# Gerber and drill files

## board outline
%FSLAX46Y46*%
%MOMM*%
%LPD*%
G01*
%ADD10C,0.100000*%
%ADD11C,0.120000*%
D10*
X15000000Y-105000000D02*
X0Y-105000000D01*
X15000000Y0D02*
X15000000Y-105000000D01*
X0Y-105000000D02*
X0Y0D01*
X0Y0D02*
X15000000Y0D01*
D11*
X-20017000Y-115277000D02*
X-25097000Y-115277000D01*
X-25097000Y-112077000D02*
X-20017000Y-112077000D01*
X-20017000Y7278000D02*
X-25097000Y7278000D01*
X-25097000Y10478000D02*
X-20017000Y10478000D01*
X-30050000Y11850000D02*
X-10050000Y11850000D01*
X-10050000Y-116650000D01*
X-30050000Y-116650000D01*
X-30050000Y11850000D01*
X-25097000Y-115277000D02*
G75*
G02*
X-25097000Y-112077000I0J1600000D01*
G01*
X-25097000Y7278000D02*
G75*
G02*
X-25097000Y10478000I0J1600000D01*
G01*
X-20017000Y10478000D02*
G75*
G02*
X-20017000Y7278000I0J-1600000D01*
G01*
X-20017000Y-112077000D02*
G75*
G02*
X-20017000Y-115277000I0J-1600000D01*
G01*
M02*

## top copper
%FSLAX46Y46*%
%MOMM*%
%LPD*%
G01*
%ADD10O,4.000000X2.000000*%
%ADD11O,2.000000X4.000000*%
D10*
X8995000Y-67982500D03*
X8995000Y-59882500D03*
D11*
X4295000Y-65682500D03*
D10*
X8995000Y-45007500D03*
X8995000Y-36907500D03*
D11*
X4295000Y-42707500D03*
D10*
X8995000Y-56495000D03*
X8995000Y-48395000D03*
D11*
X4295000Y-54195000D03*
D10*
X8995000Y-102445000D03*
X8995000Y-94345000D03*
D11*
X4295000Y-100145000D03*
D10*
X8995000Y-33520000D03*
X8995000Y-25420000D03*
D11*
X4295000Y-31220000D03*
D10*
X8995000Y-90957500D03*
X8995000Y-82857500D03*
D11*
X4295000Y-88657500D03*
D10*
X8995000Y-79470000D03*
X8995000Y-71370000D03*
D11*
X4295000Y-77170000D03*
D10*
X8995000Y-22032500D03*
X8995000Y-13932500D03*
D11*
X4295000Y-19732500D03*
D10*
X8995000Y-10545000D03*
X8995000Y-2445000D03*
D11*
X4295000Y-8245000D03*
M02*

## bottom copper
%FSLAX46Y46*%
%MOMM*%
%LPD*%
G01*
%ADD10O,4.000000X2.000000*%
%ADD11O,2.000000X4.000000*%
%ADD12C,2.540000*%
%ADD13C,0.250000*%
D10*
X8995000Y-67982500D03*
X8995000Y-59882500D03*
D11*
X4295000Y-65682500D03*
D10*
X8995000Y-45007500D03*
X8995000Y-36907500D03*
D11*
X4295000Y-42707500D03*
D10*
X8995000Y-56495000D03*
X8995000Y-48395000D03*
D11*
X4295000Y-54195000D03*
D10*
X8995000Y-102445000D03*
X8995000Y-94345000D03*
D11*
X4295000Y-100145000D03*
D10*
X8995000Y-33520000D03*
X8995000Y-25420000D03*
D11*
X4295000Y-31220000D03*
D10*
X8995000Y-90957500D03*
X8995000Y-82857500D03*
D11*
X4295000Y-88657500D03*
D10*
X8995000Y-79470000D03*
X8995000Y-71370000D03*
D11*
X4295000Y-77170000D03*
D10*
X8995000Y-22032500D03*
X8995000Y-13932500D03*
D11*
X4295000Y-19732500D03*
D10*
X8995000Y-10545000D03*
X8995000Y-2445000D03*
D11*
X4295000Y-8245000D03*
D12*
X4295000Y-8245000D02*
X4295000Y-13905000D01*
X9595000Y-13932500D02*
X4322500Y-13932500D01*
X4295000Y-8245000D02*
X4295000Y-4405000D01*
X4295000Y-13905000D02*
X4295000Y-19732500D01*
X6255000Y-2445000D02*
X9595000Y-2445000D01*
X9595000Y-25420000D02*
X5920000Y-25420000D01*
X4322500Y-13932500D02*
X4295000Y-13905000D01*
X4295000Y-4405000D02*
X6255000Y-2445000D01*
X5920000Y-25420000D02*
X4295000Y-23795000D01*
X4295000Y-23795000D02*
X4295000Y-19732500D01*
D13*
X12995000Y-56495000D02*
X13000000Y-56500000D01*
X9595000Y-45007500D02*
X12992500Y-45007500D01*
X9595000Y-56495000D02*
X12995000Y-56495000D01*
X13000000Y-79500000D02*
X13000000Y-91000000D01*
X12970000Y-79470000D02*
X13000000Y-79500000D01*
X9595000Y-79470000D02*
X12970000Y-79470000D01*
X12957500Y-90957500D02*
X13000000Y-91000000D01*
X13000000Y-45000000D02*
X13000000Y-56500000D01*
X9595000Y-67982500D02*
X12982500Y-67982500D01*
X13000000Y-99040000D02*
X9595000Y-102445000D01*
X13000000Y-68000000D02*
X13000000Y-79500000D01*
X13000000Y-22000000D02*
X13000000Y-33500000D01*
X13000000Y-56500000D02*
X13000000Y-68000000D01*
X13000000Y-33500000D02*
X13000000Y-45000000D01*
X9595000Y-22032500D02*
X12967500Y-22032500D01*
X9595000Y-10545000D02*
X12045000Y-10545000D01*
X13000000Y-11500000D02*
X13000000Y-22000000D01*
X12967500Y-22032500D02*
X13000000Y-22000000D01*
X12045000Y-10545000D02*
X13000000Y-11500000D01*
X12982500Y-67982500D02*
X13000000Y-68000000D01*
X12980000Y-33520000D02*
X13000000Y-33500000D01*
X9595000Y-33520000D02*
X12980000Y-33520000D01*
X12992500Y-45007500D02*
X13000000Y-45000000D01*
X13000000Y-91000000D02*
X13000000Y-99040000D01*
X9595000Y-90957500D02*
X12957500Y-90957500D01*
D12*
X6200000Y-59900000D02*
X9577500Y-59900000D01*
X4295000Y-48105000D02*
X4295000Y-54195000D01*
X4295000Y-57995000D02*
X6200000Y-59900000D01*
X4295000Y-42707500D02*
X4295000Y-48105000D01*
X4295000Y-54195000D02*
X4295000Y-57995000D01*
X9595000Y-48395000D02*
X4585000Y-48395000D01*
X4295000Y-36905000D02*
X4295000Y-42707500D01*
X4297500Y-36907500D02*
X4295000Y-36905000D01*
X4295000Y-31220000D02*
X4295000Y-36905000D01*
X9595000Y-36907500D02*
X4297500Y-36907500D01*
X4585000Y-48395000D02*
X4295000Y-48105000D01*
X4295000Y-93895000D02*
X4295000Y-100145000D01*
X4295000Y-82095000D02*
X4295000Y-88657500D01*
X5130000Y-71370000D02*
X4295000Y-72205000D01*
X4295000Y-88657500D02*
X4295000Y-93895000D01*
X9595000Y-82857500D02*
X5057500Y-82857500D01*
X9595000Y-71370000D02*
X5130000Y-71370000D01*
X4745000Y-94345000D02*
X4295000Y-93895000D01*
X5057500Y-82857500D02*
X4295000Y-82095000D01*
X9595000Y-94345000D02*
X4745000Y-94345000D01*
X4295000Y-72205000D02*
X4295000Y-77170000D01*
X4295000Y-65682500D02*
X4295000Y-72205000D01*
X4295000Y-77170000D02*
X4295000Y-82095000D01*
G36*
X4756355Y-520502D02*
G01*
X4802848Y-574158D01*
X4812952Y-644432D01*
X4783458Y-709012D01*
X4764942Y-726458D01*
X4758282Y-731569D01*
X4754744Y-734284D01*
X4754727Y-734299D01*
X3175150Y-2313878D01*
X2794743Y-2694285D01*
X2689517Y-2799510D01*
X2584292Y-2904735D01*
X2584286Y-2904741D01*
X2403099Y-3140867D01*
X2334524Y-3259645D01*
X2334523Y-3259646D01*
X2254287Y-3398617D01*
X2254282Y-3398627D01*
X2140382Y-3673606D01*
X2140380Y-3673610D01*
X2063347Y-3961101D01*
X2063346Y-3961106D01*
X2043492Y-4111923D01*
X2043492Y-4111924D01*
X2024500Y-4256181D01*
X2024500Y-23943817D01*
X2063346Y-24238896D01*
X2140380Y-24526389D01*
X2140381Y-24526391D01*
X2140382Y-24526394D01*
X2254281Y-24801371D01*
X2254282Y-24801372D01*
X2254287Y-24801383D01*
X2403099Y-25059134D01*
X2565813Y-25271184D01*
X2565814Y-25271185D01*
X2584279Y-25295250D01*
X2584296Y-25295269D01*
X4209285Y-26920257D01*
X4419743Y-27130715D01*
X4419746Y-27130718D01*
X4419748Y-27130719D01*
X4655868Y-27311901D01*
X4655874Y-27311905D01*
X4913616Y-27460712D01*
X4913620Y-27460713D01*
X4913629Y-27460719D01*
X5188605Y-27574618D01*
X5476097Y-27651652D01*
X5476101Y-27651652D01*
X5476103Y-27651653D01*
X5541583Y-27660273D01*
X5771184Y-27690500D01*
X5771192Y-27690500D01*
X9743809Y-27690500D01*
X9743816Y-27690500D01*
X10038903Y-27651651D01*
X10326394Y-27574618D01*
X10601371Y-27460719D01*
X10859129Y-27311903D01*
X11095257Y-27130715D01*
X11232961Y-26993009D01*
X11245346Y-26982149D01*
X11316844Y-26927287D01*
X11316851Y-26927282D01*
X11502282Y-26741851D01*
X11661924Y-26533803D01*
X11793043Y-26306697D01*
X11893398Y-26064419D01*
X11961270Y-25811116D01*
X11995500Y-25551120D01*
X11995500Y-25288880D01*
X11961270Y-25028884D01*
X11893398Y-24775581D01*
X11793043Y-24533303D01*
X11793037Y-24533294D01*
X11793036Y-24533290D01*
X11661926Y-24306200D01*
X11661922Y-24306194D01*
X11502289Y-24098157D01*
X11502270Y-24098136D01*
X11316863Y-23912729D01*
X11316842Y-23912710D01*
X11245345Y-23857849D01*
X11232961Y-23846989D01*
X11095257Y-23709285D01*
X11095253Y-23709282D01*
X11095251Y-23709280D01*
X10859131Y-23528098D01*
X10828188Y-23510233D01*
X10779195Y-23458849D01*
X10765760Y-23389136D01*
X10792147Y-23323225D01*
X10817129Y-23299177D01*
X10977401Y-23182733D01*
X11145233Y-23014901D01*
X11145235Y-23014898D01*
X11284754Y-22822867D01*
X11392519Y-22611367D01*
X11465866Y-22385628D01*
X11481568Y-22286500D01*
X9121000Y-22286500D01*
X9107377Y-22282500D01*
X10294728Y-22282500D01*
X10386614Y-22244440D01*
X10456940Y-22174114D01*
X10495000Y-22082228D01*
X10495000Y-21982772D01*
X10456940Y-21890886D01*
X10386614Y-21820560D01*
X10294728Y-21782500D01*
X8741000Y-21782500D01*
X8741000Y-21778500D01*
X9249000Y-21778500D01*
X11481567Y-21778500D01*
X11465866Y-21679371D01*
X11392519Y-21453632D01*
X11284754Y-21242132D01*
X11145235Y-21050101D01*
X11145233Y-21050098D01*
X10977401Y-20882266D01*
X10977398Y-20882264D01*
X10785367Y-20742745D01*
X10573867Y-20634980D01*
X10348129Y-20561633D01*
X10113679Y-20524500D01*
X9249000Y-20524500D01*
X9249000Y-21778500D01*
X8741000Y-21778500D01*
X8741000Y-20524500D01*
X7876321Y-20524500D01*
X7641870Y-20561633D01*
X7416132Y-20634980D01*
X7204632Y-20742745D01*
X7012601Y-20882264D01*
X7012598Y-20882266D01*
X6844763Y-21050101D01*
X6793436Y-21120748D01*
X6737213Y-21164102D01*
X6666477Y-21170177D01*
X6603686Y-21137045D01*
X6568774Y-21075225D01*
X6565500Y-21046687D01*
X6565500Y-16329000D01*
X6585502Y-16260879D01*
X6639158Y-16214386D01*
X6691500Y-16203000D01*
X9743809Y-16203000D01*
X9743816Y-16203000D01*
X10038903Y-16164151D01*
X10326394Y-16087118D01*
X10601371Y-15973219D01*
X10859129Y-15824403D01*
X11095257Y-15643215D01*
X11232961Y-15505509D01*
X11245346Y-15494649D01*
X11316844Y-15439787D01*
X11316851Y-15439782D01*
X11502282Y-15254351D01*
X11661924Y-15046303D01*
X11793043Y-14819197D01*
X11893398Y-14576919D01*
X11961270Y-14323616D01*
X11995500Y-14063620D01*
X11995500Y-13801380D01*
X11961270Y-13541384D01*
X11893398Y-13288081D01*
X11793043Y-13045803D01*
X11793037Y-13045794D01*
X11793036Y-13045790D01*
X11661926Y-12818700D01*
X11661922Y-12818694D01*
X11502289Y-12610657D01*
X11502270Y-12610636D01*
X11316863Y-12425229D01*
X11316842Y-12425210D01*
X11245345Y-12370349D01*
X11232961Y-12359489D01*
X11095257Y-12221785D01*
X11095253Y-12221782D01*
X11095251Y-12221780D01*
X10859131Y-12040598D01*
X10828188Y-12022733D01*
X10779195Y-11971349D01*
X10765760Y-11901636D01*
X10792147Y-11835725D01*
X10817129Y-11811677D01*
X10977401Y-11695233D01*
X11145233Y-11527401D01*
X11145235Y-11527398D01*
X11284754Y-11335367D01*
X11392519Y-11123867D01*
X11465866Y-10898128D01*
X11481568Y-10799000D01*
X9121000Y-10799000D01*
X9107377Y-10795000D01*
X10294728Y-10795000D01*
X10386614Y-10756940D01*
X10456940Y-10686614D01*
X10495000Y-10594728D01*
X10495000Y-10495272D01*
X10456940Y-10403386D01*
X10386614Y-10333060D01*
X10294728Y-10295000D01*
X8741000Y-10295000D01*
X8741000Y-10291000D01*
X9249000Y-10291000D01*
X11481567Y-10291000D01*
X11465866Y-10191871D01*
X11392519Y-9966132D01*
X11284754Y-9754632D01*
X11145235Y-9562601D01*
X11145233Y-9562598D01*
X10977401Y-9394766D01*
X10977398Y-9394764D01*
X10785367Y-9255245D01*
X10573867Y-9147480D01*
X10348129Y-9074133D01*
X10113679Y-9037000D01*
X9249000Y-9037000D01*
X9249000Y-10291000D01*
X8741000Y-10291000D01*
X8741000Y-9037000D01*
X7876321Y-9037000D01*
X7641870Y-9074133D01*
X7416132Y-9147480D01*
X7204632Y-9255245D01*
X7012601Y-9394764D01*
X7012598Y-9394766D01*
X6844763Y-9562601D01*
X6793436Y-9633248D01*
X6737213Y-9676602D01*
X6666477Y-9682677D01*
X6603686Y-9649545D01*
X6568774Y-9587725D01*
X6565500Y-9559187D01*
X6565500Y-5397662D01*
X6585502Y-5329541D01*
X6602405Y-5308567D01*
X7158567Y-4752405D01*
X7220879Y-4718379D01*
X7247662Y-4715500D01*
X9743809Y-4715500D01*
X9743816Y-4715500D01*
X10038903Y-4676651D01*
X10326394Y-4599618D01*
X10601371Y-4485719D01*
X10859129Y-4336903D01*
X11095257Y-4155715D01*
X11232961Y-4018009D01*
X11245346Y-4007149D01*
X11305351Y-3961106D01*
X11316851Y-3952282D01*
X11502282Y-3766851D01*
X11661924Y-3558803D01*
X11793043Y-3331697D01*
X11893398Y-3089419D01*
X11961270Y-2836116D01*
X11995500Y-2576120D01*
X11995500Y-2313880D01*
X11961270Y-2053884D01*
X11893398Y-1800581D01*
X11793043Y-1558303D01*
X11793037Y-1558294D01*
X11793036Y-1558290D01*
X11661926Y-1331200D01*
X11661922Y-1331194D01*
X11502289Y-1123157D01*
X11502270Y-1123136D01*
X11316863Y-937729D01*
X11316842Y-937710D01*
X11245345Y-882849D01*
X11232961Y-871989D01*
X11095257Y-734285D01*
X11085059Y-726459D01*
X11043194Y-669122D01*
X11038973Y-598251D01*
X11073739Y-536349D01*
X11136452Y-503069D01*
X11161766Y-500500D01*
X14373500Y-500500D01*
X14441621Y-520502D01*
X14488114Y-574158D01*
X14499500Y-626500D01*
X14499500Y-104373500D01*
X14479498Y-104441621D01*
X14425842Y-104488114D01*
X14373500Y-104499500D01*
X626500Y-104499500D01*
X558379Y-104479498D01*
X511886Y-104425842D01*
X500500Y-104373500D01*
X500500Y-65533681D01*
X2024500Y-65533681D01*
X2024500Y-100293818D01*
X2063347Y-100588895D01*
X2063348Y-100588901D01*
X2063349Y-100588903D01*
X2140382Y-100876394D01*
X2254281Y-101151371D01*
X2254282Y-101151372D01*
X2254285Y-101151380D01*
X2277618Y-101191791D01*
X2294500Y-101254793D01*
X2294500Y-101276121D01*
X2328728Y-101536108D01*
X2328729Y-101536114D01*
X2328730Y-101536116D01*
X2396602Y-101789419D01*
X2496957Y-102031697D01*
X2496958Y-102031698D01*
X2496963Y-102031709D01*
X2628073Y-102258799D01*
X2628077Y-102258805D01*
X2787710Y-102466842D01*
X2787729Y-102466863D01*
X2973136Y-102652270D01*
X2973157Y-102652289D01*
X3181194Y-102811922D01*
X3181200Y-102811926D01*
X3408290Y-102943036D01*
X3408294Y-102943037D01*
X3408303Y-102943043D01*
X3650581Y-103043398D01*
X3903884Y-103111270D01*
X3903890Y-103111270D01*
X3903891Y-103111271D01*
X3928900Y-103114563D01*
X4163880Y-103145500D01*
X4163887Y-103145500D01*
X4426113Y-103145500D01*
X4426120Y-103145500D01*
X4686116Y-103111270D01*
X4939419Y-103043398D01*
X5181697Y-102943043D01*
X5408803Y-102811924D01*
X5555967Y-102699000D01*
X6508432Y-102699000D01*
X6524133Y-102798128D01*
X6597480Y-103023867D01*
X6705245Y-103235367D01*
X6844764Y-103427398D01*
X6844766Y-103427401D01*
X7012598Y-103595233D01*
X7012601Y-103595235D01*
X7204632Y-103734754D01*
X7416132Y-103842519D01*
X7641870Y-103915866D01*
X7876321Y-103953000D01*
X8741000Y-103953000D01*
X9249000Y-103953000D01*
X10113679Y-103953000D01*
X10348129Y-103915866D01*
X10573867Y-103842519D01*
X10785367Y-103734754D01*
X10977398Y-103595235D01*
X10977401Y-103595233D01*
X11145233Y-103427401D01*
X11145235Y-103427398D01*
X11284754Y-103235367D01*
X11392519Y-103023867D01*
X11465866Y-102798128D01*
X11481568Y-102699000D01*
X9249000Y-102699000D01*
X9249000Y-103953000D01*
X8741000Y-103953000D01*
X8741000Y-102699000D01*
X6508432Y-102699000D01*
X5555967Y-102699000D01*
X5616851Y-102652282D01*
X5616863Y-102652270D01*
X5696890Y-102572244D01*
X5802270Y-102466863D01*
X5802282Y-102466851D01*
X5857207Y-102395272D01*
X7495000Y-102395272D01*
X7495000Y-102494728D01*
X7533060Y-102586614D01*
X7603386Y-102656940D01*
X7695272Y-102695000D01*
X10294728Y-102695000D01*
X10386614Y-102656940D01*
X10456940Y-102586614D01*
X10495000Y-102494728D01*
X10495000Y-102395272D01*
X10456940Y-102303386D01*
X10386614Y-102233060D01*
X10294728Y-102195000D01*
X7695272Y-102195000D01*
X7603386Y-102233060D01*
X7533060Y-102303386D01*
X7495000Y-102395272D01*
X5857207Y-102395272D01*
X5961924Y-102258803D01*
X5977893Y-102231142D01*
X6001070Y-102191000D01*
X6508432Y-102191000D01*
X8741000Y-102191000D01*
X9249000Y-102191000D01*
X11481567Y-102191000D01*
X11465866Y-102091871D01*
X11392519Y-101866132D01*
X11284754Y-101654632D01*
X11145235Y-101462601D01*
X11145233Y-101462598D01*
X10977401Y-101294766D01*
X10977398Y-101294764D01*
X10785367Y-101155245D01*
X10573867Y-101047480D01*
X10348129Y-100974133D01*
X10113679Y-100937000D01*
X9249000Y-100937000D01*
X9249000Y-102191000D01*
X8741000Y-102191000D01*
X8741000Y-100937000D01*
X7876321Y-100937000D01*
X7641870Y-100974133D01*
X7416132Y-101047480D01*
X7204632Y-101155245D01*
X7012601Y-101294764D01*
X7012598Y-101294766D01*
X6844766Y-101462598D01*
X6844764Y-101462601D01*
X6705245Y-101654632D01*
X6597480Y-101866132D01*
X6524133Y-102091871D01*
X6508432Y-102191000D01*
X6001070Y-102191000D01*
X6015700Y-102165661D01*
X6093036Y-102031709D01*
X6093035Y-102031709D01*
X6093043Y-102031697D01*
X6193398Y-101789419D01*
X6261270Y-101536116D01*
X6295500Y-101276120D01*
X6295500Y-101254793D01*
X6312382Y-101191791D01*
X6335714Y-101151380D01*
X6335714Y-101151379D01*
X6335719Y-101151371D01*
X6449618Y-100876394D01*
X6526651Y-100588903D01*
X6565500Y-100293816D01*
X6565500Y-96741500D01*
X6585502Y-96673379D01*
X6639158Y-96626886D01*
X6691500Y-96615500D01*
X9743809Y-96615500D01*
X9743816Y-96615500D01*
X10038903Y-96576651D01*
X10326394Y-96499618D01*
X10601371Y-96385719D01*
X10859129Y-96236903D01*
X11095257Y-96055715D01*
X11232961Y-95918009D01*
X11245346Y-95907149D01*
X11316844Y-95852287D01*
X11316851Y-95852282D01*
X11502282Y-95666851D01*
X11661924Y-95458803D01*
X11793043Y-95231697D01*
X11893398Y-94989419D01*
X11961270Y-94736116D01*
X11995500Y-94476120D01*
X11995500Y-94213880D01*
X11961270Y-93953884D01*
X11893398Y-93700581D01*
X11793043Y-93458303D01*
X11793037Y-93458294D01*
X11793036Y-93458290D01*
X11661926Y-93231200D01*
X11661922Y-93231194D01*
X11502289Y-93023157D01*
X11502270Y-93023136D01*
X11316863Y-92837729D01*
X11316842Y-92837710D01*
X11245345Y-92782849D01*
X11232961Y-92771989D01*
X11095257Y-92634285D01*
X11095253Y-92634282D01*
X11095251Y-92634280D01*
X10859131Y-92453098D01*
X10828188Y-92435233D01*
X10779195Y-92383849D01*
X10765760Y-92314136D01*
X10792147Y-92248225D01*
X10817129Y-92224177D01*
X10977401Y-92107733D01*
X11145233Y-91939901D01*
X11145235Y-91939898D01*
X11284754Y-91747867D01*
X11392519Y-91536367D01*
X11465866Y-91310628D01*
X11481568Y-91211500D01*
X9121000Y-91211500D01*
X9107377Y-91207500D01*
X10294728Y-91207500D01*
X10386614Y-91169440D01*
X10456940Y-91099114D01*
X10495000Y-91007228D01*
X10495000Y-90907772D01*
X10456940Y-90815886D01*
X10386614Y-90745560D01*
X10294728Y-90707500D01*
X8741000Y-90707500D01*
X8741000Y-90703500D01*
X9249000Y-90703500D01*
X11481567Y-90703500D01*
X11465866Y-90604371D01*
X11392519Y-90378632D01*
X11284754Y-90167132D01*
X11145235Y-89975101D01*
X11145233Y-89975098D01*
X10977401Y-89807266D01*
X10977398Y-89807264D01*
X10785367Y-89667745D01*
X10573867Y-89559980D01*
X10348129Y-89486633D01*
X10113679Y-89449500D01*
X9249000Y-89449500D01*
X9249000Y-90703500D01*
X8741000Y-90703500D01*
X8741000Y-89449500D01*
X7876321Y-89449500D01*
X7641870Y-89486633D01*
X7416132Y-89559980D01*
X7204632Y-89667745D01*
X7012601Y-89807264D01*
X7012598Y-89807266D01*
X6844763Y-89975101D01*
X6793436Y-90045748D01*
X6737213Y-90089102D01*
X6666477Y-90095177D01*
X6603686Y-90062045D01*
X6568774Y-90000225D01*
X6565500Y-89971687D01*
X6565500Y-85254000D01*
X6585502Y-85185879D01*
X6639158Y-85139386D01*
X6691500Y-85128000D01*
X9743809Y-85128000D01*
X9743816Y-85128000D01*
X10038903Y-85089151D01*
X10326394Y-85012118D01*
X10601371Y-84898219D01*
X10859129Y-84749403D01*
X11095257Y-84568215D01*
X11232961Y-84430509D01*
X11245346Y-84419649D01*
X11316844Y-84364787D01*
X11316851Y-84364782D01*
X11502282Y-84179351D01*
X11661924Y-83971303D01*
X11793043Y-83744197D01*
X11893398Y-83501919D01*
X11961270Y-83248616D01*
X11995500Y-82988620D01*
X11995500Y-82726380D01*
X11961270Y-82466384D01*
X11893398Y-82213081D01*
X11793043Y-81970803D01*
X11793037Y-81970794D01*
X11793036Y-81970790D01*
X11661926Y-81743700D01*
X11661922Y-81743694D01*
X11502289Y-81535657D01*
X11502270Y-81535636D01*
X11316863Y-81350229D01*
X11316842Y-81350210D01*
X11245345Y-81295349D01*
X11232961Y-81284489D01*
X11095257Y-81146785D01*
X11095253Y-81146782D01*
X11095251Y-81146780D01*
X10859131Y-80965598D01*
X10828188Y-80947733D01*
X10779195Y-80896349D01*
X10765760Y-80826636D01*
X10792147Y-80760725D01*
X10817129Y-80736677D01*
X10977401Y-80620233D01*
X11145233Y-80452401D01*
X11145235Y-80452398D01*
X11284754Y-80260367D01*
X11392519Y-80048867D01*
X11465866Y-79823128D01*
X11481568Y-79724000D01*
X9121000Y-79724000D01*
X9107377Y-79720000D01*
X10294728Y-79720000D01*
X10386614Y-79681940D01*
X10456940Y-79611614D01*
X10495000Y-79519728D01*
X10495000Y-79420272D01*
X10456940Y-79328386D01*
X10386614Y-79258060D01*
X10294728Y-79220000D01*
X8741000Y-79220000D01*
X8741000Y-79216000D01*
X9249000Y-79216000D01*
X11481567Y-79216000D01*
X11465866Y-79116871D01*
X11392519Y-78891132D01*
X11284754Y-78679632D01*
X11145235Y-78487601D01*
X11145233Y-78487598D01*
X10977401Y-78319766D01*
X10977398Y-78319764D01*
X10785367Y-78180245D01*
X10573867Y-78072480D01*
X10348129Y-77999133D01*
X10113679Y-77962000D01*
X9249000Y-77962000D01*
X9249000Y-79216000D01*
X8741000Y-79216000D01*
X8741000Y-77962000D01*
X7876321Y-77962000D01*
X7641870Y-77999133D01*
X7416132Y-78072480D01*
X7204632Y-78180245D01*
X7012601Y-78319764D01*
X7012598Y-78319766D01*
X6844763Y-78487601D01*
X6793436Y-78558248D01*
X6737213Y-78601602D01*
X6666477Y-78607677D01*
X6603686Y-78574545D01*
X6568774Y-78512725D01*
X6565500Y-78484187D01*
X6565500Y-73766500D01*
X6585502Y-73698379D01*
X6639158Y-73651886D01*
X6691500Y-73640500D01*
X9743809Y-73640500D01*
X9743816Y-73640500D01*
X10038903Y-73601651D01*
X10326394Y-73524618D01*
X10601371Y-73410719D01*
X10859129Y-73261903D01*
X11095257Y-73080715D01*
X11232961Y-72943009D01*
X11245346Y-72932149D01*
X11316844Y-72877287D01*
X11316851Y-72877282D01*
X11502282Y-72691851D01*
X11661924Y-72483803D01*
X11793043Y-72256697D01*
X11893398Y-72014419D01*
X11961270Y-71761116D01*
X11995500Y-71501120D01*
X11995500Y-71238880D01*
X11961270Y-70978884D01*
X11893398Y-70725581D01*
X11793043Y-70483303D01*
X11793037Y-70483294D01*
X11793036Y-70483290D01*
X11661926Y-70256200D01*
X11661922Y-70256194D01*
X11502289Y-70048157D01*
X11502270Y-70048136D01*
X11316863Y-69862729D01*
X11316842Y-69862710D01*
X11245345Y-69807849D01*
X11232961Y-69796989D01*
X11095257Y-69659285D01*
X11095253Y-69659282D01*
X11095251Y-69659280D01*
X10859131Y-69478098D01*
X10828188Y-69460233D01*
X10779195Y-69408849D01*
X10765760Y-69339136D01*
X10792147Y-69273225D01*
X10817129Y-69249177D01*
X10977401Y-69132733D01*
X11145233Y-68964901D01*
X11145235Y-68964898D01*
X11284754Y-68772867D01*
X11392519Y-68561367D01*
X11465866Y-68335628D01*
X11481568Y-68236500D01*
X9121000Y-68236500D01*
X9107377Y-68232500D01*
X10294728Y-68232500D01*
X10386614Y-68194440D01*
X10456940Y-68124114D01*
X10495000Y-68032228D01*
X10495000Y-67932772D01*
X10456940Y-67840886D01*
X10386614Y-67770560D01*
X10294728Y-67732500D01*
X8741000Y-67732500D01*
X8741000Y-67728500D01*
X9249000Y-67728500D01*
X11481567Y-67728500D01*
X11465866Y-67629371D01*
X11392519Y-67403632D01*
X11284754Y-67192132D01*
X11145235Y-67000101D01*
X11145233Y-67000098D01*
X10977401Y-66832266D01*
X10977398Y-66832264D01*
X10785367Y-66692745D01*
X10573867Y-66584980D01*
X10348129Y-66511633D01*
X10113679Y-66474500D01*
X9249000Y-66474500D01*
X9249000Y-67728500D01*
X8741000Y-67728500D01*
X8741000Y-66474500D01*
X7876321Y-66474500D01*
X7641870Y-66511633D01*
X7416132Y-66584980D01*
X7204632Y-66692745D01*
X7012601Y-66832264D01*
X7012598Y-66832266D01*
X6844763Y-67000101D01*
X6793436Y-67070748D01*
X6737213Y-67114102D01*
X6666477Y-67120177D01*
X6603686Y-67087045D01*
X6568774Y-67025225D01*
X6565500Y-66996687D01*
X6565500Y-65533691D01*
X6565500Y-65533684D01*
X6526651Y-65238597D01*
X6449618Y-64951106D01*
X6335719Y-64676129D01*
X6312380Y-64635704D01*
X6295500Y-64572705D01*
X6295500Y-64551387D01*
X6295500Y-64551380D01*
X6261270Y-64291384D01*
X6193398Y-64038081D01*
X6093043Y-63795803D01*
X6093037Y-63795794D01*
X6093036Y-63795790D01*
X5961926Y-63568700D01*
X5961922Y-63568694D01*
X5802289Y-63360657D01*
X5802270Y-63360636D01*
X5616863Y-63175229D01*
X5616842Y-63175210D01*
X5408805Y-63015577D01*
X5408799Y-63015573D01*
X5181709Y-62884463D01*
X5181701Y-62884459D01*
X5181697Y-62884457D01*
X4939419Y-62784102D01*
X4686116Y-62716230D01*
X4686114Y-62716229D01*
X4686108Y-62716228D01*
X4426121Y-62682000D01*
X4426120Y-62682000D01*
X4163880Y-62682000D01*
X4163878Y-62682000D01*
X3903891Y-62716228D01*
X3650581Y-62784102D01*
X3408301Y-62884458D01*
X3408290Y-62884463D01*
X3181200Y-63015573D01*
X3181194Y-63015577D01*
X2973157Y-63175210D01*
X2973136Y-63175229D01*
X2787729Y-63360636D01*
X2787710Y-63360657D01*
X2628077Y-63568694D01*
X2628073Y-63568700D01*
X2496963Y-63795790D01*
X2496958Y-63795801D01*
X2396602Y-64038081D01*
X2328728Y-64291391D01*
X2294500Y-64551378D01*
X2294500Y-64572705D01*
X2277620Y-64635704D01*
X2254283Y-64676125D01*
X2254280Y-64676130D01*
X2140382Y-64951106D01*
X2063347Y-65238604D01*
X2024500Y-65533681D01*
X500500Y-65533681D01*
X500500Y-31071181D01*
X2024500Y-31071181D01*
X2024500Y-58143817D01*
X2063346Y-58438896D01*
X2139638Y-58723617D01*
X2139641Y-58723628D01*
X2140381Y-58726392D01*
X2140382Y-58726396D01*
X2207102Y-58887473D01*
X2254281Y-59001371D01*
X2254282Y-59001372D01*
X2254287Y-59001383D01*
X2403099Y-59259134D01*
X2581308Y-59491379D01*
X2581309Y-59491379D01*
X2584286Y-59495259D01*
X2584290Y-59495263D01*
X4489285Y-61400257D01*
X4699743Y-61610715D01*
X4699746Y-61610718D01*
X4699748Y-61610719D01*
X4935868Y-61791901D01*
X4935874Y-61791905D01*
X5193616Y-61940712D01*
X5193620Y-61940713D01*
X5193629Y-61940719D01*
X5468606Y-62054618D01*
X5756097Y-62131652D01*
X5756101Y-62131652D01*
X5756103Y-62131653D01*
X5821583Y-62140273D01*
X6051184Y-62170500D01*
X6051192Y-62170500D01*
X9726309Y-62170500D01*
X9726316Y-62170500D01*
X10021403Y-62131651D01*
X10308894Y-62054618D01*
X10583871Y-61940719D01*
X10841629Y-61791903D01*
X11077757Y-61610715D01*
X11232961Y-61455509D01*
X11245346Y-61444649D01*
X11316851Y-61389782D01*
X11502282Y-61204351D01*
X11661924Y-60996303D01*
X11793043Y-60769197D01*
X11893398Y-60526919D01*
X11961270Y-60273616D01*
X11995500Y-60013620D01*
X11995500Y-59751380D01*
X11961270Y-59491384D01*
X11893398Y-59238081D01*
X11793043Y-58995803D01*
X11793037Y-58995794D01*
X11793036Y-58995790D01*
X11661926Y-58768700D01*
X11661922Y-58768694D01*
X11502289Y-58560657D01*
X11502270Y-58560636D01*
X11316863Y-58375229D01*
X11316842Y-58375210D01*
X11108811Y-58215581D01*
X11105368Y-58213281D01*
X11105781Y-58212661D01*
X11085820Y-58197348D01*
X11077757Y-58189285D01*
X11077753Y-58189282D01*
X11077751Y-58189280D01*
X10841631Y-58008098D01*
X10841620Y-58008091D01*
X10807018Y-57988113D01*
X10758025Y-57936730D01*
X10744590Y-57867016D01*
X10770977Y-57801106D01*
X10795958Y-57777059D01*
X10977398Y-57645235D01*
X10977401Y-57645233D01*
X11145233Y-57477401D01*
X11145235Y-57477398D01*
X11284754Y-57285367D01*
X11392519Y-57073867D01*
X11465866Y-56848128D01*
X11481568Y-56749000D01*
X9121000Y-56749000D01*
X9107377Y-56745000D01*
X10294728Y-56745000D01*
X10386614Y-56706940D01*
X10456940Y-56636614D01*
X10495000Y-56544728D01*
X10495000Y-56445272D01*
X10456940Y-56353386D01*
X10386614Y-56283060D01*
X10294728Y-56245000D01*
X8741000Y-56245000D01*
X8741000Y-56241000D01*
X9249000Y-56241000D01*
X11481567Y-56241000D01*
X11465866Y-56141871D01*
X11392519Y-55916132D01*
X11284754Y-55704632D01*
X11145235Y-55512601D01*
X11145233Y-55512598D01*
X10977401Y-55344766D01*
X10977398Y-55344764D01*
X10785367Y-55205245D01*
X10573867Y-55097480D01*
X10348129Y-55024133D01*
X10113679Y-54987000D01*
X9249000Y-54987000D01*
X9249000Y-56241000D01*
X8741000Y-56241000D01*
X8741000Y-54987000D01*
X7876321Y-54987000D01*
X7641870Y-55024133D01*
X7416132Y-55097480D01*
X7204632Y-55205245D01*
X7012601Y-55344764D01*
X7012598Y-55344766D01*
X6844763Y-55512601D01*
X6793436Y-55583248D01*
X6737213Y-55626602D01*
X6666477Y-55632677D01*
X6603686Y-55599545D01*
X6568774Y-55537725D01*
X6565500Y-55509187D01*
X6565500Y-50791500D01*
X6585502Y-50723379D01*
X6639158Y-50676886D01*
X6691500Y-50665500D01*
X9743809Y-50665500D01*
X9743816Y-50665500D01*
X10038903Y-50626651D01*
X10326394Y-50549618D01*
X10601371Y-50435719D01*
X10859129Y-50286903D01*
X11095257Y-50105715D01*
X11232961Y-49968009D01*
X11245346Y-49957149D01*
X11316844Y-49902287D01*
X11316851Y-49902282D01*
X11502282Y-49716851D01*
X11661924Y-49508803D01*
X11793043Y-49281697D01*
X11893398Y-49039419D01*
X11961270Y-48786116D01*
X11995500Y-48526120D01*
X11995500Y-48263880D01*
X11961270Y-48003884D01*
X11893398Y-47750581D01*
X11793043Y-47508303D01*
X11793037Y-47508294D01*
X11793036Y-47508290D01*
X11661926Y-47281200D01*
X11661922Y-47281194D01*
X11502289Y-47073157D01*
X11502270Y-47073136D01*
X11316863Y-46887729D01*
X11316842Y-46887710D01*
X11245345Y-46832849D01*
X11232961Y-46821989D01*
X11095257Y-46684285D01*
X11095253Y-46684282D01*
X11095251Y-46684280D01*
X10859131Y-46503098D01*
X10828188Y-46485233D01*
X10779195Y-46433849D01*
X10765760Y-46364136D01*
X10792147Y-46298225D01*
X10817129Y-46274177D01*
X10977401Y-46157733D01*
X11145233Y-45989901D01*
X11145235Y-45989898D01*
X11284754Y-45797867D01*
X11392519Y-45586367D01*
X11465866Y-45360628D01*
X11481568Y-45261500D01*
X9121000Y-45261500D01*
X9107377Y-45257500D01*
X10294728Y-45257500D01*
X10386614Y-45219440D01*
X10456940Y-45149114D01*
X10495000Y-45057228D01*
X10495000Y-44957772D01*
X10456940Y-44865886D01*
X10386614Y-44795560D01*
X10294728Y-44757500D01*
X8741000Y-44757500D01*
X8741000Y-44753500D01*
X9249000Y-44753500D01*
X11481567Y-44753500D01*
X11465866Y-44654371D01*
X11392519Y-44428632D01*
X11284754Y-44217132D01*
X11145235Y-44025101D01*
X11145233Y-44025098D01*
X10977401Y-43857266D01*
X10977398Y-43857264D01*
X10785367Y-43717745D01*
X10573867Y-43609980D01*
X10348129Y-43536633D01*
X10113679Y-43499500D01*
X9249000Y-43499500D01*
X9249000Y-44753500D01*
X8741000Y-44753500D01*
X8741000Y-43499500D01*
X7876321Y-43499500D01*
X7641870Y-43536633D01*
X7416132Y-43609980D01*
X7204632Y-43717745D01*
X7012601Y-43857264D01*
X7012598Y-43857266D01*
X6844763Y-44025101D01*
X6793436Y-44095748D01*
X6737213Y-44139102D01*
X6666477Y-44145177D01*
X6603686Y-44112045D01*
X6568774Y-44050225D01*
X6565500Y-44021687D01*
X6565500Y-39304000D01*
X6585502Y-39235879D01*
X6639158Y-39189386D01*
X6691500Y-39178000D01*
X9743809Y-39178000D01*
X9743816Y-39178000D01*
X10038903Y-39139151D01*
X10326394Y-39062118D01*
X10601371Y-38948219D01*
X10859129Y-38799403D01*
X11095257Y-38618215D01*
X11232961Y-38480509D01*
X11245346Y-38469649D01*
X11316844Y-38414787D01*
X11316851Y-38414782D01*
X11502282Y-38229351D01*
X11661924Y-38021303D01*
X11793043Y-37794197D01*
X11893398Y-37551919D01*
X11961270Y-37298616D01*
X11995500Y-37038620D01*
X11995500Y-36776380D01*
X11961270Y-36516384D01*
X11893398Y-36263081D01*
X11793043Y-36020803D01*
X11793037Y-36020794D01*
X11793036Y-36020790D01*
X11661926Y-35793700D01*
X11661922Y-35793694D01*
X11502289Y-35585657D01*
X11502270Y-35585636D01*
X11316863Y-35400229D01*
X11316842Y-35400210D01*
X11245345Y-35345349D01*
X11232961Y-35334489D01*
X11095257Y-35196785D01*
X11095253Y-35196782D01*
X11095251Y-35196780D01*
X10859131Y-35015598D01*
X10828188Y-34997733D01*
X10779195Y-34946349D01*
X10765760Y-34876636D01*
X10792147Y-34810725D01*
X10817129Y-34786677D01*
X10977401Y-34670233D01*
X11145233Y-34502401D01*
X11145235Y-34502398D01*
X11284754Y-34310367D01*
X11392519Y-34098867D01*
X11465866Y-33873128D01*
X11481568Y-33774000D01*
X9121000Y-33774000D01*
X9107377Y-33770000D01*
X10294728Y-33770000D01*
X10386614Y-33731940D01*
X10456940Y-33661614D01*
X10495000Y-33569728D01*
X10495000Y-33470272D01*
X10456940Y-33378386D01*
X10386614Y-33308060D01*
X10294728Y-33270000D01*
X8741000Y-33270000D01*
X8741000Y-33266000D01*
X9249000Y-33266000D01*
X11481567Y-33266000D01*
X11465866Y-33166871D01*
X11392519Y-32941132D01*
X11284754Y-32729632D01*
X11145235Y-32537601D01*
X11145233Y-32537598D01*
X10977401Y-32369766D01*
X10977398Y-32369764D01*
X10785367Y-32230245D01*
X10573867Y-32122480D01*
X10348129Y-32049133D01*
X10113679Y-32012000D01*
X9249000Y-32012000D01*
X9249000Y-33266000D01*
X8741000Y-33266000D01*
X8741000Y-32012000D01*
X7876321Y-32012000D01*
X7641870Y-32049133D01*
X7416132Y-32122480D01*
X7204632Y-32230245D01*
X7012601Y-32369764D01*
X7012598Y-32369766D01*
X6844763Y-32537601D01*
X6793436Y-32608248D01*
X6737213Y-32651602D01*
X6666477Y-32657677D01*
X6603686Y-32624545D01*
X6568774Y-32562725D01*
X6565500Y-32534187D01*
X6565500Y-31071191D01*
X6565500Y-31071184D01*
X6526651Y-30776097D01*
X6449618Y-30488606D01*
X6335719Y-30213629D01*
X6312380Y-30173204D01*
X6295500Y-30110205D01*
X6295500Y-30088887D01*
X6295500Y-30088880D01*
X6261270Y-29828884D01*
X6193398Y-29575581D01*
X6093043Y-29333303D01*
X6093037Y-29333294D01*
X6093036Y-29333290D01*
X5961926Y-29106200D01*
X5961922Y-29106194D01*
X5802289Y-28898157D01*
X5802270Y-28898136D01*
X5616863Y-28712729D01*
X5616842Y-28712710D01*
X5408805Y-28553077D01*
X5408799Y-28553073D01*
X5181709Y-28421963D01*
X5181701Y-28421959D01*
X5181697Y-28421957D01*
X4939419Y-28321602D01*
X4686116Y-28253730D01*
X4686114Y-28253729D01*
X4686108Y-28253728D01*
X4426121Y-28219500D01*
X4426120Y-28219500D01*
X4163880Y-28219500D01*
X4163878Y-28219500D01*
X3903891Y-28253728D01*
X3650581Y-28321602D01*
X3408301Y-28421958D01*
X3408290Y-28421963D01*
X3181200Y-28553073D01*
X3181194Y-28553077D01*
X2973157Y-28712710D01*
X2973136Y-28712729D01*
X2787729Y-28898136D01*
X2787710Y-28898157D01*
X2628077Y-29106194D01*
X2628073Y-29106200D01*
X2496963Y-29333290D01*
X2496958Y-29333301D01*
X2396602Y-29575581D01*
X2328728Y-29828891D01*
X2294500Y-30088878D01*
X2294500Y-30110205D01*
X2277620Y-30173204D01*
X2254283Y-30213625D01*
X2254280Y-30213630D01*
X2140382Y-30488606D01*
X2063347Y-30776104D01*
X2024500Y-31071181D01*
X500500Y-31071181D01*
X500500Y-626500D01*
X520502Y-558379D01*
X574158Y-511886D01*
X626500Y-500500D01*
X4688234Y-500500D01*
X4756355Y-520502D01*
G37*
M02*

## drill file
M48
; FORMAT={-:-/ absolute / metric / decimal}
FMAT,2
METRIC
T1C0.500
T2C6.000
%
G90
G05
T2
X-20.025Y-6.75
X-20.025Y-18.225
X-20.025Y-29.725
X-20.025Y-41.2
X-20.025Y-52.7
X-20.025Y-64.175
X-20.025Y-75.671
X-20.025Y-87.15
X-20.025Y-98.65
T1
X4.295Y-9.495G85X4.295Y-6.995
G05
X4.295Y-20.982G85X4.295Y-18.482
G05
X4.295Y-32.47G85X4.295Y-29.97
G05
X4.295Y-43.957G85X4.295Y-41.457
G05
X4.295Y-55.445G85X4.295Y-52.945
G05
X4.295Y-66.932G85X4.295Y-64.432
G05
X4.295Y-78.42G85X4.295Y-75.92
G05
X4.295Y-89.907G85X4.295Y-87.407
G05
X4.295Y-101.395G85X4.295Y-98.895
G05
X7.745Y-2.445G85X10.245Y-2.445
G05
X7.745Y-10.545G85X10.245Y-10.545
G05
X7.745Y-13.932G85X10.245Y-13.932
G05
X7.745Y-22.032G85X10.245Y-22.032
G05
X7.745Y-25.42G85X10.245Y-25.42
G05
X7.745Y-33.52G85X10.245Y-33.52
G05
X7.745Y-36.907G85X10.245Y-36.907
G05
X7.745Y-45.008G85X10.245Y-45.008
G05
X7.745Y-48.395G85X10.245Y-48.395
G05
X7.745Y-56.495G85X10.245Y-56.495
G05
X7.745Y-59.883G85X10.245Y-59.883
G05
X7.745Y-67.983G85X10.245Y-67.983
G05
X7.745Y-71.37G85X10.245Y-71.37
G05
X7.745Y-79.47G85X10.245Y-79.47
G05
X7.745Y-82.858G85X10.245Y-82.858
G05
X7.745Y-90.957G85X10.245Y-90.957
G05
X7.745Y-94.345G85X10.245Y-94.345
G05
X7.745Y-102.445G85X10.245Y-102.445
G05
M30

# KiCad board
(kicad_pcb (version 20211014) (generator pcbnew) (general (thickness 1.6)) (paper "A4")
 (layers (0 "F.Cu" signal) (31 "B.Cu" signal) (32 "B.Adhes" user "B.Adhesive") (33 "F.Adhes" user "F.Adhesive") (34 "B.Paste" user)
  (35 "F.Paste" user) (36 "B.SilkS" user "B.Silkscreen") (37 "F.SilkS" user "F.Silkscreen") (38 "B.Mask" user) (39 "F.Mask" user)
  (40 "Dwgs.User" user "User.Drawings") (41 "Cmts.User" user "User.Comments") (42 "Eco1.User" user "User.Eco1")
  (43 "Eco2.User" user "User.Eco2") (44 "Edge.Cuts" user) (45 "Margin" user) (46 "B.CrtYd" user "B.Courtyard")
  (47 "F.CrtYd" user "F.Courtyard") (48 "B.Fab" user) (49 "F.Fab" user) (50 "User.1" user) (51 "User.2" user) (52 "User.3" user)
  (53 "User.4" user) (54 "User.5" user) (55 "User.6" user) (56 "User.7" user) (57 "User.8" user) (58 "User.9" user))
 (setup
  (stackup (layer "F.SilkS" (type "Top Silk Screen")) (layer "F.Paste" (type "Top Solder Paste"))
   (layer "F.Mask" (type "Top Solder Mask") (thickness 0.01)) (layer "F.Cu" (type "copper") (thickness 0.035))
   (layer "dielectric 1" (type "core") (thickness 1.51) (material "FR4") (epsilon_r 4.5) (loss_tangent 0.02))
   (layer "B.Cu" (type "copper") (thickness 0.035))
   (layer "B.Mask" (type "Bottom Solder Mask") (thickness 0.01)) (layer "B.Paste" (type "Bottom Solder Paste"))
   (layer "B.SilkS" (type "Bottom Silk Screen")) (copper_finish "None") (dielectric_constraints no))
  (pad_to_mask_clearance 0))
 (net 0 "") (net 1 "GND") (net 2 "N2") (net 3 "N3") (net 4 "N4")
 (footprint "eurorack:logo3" (layer "F.Cu") (at -25.575 54.775 90)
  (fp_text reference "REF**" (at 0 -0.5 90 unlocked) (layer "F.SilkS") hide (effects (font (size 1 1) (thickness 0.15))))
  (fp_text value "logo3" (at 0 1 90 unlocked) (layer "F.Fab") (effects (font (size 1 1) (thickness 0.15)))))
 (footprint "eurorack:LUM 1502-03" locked (layer "F.Cu") (at 2.895 58.4825)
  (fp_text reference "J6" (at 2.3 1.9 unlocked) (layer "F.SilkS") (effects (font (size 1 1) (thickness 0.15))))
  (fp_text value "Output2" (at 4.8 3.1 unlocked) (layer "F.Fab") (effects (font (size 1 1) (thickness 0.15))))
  (pad "S" thru_hole oval locked (at 6.1 9.5) (size 4 2) (drill oval 3 0.5) (layers *.Cu *.Mask) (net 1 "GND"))
  (pad "T" thru_hole oval locked (at 6.1 1.4) (size 4 2) (drill oval 3 0.5) (layers *.Cu *.Mask) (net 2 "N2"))
  (pad "TN" thru_hole oval locked (at 1.4 7.2 90) (size 4 2) (drill oval 3 0.5) (layers *.Cu *.Mask) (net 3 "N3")))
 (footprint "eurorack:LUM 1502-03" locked (layer "F.Cu") (at 2.895 35.5075)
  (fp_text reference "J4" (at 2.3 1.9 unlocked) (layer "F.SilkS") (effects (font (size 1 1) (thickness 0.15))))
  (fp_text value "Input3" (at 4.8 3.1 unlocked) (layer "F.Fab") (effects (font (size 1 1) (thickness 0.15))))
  (pad "S" thru_hole oval locked (at 6.1 9.5) (size 4 2) (drill oval 3 0.5) (layers *.Cu *.Mask) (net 1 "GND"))
  (pad "T" thru_hole oval locked (at 6.1 1.4) (size 4 2) (drill oval 3 0.5) (layers *.Cu *.Mask) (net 2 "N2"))
  (pad "TN" thru_hole oval locked (at 1.4 7.2 90) (size 4 2) (drill oval 3 0.5) (layers *.Cu *.Mask) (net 2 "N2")))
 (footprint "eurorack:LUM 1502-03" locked (layer "F.Cu") (at 2.895 46.995)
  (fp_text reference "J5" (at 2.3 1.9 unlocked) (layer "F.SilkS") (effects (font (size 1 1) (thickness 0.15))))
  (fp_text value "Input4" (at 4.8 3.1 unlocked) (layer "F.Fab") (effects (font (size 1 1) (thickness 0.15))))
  (pad "S" thru_hole oval locked (at 6.1 9.5) (size 4 2) (drill oval 3 0.5) (layers *.Cu *.Mask) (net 1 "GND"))
  (pad "T" thru_hole oval locked (at 6.1 1.4) (size 4 2) (drill oval 3 0.5) (layers *.Cu *.Mask) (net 2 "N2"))
  (pad "TN" thru_hole oval locked (at 1.4 7.2 90) (size 4 2) (drill oval 3 0.5) (layers *.Cu *.Mask) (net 2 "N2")))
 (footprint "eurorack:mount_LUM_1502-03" (layer "F.Cu") (at -20.025 41.2)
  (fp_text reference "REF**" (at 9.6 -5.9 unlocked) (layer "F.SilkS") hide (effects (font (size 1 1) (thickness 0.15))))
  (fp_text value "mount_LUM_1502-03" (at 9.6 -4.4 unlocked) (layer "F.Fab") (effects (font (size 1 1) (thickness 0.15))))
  (pad "" np_thru_hole circle (at 0 0) (size 6 6) (drill 6) (layers F&B.Cu *.Mask)))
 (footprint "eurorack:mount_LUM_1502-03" (layer "F.Cu") (at -20.025 52.7)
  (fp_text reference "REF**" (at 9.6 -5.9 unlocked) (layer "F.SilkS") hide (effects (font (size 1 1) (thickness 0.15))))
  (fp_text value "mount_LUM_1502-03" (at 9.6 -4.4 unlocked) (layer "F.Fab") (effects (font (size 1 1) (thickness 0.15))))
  (pad "" np_thru_hole circle (at 0 0) (size 6 6) (drill 6) (layers F&B.Cu *.Mask)))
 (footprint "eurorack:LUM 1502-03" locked (layer "F.Cu") (at 2.895 92.945)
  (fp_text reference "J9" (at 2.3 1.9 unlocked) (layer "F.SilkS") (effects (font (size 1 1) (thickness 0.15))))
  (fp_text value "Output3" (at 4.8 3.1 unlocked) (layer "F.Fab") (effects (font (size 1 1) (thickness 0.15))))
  (pad "S" thru_hole oval locked (at 6.1 9.5) (size 4 2) (drill oval 3 0.5) (layers *.Cu *.Mask) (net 1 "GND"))
  (pad "T" thru_hole oval locked (at 6.1 1.4) (size 4 2) (drill oval 3 0.5) (layers *.Cu *.Mask) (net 3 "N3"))
  (pad "TN" thru_hole oval locked (at 1.4 7.2 90) (size 4 2) (drill oval 3 0.5) (layers *.Cu *.Mask) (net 3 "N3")))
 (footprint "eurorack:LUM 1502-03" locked (layer "F.Cu") (at 2.895 24.02)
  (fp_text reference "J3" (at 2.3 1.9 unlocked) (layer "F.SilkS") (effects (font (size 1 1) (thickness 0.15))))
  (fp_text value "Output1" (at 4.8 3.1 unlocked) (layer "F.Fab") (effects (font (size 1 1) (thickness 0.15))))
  (pad "S" thru_hole oval locked (at 6.1 9.5) (size 4 2) (drill oval 3 0.5) (layers *.Cu *.Mask) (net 1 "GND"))
  (pad "T" thru_hole oval locked (at 6.1 1.4) (size 4 2) (drill oval 3 0.5) (layers *.Cu *.Mask) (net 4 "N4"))
  (pad "TN" thru_hole oval locked (at 1.4 7.2 90) (size 4 2) (drill oval 3 0.5) (layers *.Cu *.Mask) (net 2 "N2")))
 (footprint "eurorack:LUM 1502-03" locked (layer "F.Cu") (at 2.895 81.4575)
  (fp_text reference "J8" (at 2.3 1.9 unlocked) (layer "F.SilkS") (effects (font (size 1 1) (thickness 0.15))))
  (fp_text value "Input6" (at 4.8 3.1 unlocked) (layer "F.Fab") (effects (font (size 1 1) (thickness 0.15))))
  (pad "S" thru_hole oval locked (at 6.1 9.5) (size 4 2) (drill oval 3 0.5) (layers *.Cu *.Mask) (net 1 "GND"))
  (pad "T" thru_hole oval locked (at 6.1 1.4) (size 4 2) (drill oval 3 0.5) (layers *.Cu *.Mask) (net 3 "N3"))
  (pad "TN" thru_hole oval locked (at 1.4 7.2 90) (size 4 2) (drill oval 3 0.5) (layers *.Cu *.Mask) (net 3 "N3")))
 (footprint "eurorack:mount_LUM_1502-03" (layer "F.Cu") (at -20.025 64.175)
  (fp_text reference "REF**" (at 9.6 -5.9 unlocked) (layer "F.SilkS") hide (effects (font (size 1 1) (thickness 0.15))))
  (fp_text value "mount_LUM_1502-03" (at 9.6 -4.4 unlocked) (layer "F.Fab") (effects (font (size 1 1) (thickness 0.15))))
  (pad "" np_thru_hole circle (at 0 0) (size 6 6) (drill 6) (layers F&B.Cu *.Mask)))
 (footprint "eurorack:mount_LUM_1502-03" (layer "F.Cu") (at -20.025 6.75)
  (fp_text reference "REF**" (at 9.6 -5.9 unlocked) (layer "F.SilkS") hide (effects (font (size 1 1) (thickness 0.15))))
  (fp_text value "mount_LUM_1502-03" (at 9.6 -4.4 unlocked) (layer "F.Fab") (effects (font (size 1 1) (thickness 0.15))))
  (pad "" np_thru_hole circle (at 0 0) (size 6 6) (drill 6) (layers F&B.Cu *.Mask)))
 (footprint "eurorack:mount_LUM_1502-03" (layer "F.Cu") (at -20.025 75.671059)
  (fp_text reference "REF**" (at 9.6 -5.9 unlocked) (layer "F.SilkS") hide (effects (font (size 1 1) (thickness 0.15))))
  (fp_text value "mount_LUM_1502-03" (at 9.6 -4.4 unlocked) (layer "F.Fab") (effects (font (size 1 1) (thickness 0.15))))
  (pad "" np_thru_hole circle (at 0 0) (size 6 6) (drill 6) (layers F&B.Cu *.Mask)))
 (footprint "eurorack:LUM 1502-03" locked (layer "F.Cu") (at 2.895 69.97)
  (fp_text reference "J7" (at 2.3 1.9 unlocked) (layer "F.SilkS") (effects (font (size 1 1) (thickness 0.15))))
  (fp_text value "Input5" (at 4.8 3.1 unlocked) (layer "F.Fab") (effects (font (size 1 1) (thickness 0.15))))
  (pad "S" thru_hole oval locked (at 6.1 9.5) (size 4 2) (drill oval 3 0.5) (layers *.Cu *.Mask) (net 1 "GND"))
  (pad "T" thru_hole oval locked (at 6.1 1.4) (size 4 2) (drill oval 3 0.5) (layers *.Cu *.Mask) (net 3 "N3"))
  (pad "TN" thru_hole oval locked (at 1.4 7.2 90) (size 4 2) (drill oval 3 0.5) (layers *.Cu *.Mask) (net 3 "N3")))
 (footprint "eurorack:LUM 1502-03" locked (layer "F.Cu") (at 2.895 12.5325)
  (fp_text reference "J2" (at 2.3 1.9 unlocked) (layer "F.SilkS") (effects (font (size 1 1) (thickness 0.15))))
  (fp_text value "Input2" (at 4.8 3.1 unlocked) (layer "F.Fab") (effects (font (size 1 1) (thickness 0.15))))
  (pad "S" thru_hole oval locked (at 6.1 9.5) (size 4 2) (drill oval 3 0.5) (layers *.Cu *.Mask) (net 1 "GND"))
  (pad "T" thru_hole oval locked (at 6.1 1.4) (size 4 2) (drill oval 3 0.5) (layers *.Cu *.Mask) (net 4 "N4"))
  (pad "TN" thru_hole oval locked (at 1.4 7.2 90) (size 4 2) (drill oval 3 0.5) (layers *.Cu *.Mask) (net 4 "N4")))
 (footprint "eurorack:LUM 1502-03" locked (layer "F.Cu") (at 2.895 1.045)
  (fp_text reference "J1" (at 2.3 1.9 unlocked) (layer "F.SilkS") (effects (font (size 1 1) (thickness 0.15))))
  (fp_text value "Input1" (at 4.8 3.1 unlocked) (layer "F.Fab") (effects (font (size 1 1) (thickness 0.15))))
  (pad "S" thru_hole oval locked (at 6.1 9.5) (size 4 2) (drill oval 3 0.5) (layers *.Cu *.Mask) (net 1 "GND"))
  (pad "T" thru_hole oval locked (at 6.1 1.4) (size 4 2) (drill oval 3 0.5) (layers *.Cu *.Mask) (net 4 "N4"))
  (pad "TN" thru_hole oval locked (at 1.4 7.2 90) (size 4 2) (drill oval 3 0.5) (layers *.Cu *.Mask) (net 4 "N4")))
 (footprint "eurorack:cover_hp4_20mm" (layer "F.Cu") (at -30.05 -11.85)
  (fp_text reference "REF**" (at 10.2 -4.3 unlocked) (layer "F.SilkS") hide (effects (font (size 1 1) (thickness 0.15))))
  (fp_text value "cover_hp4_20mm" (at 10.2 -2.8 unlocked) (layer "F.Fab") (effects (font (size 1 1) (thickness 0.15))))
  (fp_line (start 10.033 127.127) (end 4.953 127.127) (layer "Edge.Cuts") (width 0.12))
  (fp_line (start 4.953 123.927) (end 10.033 123.927) (layer "Edge.Cuts") (width 0.12))
  (fp_line (start 10.033 4.572) (end 4.953 4.572) (layer "Edge.Cuts") (width 0.12))
  (fp_line (start 4.953 1.372) (end 10.033 1.372) (layer "Edge.Cuts") (width 0.12))
  (fp_rect (start 0 0) (end 20 128.5) (layer "Edge.Cuts") (width 0.12) (fill none))
  (fp_arc (start 4.953 127.127) (mid 3.353 125.527) (end 4.953 123.927) (layer "Edge.Cuts") (width 0.12))
  (fp_arc (start 4.953 4.572) (mid 3.353 2.972) (end 4.953 1.372) (layer "Edge.Cuts") (width 0.12))
  (fp_arc (start 10.033 1.372) (mid 11.633 2.972) (end 10.033 4.572) (layer "Edge.Cuts") (width 0.12))
  (fp_arc (start 10.033 123.927) (mid 11.633 125.527) (end 10.033 127.127) (layer "Edge.Cuts") (width 0.12)))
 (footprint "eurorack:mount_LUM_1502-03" (layer "F.Cu") (at -20.025 98.65)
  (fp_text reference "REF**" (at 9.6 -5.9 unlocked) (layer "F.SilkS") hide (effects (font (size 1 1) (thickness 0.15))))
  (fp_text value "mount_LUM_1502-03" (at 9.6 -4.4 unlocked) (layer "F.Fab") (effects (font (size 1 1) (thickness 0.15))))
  (pad "" np_thru_hole circle (at 0 0) (size 6 6) (drill 6) (layers F&B.Cu *.Mask)))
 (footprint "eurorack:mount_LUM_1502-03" (layer "F.Cu") (at -20.025 18.225)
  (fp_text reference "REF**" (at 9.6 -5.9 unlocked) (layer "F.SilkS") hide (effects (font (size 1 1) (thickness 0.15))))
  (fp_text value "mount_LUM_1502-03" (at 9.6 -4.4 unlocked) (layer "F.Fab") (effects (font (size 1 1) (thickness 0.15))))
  (pad "" np_thru_hole circle (at 0 0) (size 6 6) (drill 6) (layers F&B.Cu *.Mask)))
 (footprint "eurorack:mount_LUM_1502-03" (layer "F.Cu") (at -20.025 87.15)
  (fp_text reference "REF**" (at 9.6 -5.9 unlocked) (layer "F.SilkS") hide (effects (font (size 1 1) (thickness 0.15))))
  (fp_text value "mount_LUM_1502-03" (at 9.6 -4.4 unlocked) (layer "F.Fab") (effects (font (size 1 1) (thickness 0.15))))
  (pad "" np_thru_hole circle (at 0 0) (size 6 6) (drill 6) (layers F&B.Cu *.Mask)))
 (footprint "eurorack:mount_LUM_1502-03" (layer "F.Cu") (at -20.025 29.725)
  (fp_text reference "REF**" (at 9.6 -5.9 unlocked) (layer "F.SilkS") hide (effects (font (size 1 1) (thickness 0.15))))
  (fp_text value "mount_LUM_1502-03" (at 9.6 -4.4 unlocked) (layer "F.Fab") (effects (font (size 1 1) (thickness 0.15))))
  (pad "" np_thru_hole circle (at 0 0) (size 6 6) (drill 6) (layers F&B.Cu *.Mask)))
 (gr_line locked (start 15 105) (end 0 105) (layer "Edge.Cuts") (width 0.1))
 (gr_line locked (start 15 0) (end 15 105) (layer "Edge.Cuts") (width 0.1))
 (gr_line locked (start 0 105) (end 0 0) (layer "Edge.Cuts") (width 0.1))
 (gr_line locked (start 0 0) (end 15 0) (layer "Edge.Cuts") (width 0.1))
 (segment locked (start 4.295 8.245) (end 4.295 13.905) (width 2.54) (layer "B.Cu") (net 4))
 (segment locked (start 9.595 13.9325) (end 4.3225 13.9325) (width 2.54) (layer "B.Cu") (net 4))
 (segment locked (start 4.295 8.245) (end 4.295 4.405) (width 2.54) (layer "B.Cu") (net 4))
 (segment locked (start 4.295 13.905) (end 4.295 19.7325) (width 2.54) (layer "B.Cu") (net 4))
 (segment locked (start 6.255 2.445) (end 9.595 2.445) (width 2.54) (layer "B.Cu") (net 4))
 (segment locked (start 9.595 25.42) (end 5.92 25.42) (width 2.54) (layer "B.Cu") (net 4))
 (segment locked (start 4.3225 13.9325) (end 4.295 13.905) (width 2.54) (layer "B.Cu") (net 4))
 (segment locked (start 4.295 4.405) (end 6.255 2.445) (width 2.54) (layer "B.Cu") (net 4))
 (segment locked (start 5.92 25.42) (end 4.295 23.795) (width 2.54) (layer "B.Cu") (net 4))
 (segment locked (start 4.295 23.795) (end 4.295 19.7325) (width 2.54) (layer "B.Cu") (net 4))
 (segment locked (start 12.995 56.495) (end 13 56.5) (width 0.25) (layer "B.Cu") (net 1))
 (segment locked (start 9.595 45.0075) (end 12.9925 45.0075) (width 0.25) (layer "B.Cu") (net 1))
 (segment locked (start 9.595 56.495) (end 12.995 56.495) (width 0.25) (layer "B.Cu") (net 1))
 (segment locked (start 13 79.5) (end 13 91) (width 0.25) (layer "B.Cu") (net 1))
 (segment locked (start 12.97 79.47) (end 13 79.5) (width 0.25) (layer "B.Cu") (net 1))
 (segment locked (start 9.595 79.47) (end 12.97 79.47) (width 0.25) (layer "B.Cu") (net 1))
 (segment locked (start 12.9575 90.9575) (end 13 91) (width 0.25) (layer "B.Cu") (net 1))
 (segment locked (start 13 45) (end 13 56.5) (width 0.25) (layer "B.Cu") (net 1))
 (segment locked (start 9.595 67.9825) (end 12.9825 67.9825) (width 0.25) (layer "B.Cu") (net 1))
 (segment locked (start 13 99.04) (end 9.595 102.445) (width 0.25) (layer "B.Cu") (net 1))
 (segment locked (start 13 68) (end 13 79.5) (width 0.25) (layer "B.Cu") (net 1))
 (segment locked (start 13 22) (end 13 33.5) (width 0.25) (layer "B.Cu") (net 1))
 (segment locked (start 13 56.5) (end 13 68) (width 0.25) (layer "B.Cu") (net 1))
 (segment locked (start 13 33.5) (end 13 45) (width 0.25) (layer "B.Cu") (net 1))
 (segment locked (start 9.595 22.0325) (end 12.9675 22.0325) (width 0.25) (layer "B.Cu") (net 1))
 (segment locked (start 9.595 10.545) (end 12.045 10.545) (width 0.25) (layer "B.Cu") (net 1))
 (segment locked (start 13 11.5) (end 13 22) (width 0.25) (layer "B.Cu") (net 1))
 (segment locked (start 12.9675 22.0325) (end 13 22) (width 0.25) (layer "B.Cu") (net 1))
 (segment locked (start 12.045 10.545) (end 13 11.5) (width 0.25) (layer "B.Cu") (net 1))
 (segment locked (start 12.9825 67.9825) (end 13 68) (width 0.25) (layer "B.Cu") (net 1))
 (segment locked (start 12.98 33.52) (end 13 33.5) (width 0.25) (layer "B.Cu") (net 1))
 (segment locked (start 9.595 33.52) (end 12.98 33.52) (width 0.25) (layer "B.Cu") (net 1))
 (segment locked (start 12.9925 45.0075) (end 13 45) (width 0.25) (layer "B.Cu") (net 1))
 (segment locked (start 13 91) (end 13 99.04) (width 0.25) (layer "B.Cu") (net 1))
 (segment locked (start 9.595 90.9575) (end 12.9575 90.9575) (width 0.25) (layer "B.Cu") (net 1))
 (segment locked (start 6.2 59.9) (end 9.5775 59.9) (width 2.54) (layer "B.Cu") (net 2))
 (segment locked (start 4.295 48.105) (end 4.295 54.195) (width 2.54) (layer "B.Cu") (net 2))
 (segment locked (start 4.295 57.995) (end 6.2 59.9) (width 2.54) (layer "B.Cu") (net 2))
 (segment locked (start 4.295 42.7075) (end 4.295 48.105) (width 2.54) (layer "B.Cu") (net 2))
 (segment locked (start 4.295 54.195) (end 4.295 57.995) (width 2.54) (layer "B.Cu") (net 2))
 (segment locked (start 9.595 48.395) (end 4.585 48.395) (width 2.54) (layer "B.Cu") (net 2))
 (segment locked (start 4.295 36.905) (end 4.295 42.7075) (width 2.54) (layer "B.Cu") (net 2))
 (segment locked (start 4.2975 36.9075) (end 4.295 36.905) (width 2.54) (layer "B.Cu") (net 2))
 (segment locked (start 4.295 31.22) (end 4.295 36.905) (width 2.54) (layer "B.Cu") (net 2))
 (segment locked (start 9.595 36.9075) (end 4.2975 36.9075) (width 2.54) (layer "B.Cu") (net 2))
 (segment locked (start 4.585 48.395) (end 4.295 48.105) (width 2.54) (layer "B.Cu") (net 2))
 (segment locked (start 4.295 93.895) (end 4.295 100.145) (width 2.54) (layer "B.Cu") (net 3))
 (segment locked (start 4.295 82.095) (end 4.295 88.6575) (width 2.54) (layer "B.Cu") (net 3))
 (segment locked (start 5.13 71.37) (end 4.295 72.205) (width 2.54) (layer "B.Cu") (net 3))
 (segment locked (start 4.295 88.6575) (end 4.295 93.895) (width 2.54) (layer "B.Cu") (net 3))
 (segment locked (start 9.595 82.8575) (end 5.0575 82.8575) (width 2.54) (layer "B.Cu") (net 3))
 (segment locked (start 9.595 71.37) (end 5.13 71.37) (width 2.54) (layer "B.Cu") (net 3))
 (segment locked (start 4.745 94.345) (end 4.295 93.895) (width 2.54) (layer "B.Cu") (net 3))
 (segment locked (start 5.0575 82.8575) (end 4.295 82.095) (width 2.54) (layer "B.Cu") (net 3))
 (segment locked (start 9.595 94.345) (end 4.745 94.345) (width 2.54) (layer "B.Cu") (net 3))
 (segment locked (start 4.295 72.205) (end 4.295 77.17) (width 2.54) (layer "B.Cu") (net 3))
 (segment locked (start 4.295 65.6825) (end 4.295 72.205) (width 2.54) (layer "B.Cu") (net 3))
 (segment locked (start 4.295 77.17) (end 4.295 82.095) (width 2.54) (layer "B.Cu") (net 3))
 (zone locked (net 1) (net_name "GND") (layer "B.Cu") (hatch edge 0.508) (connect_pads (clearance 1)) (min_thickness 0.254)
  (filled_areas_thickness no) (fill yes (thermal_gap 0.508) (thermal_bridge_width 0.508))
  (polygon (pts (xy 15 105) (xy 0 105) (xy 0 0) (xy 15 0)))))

